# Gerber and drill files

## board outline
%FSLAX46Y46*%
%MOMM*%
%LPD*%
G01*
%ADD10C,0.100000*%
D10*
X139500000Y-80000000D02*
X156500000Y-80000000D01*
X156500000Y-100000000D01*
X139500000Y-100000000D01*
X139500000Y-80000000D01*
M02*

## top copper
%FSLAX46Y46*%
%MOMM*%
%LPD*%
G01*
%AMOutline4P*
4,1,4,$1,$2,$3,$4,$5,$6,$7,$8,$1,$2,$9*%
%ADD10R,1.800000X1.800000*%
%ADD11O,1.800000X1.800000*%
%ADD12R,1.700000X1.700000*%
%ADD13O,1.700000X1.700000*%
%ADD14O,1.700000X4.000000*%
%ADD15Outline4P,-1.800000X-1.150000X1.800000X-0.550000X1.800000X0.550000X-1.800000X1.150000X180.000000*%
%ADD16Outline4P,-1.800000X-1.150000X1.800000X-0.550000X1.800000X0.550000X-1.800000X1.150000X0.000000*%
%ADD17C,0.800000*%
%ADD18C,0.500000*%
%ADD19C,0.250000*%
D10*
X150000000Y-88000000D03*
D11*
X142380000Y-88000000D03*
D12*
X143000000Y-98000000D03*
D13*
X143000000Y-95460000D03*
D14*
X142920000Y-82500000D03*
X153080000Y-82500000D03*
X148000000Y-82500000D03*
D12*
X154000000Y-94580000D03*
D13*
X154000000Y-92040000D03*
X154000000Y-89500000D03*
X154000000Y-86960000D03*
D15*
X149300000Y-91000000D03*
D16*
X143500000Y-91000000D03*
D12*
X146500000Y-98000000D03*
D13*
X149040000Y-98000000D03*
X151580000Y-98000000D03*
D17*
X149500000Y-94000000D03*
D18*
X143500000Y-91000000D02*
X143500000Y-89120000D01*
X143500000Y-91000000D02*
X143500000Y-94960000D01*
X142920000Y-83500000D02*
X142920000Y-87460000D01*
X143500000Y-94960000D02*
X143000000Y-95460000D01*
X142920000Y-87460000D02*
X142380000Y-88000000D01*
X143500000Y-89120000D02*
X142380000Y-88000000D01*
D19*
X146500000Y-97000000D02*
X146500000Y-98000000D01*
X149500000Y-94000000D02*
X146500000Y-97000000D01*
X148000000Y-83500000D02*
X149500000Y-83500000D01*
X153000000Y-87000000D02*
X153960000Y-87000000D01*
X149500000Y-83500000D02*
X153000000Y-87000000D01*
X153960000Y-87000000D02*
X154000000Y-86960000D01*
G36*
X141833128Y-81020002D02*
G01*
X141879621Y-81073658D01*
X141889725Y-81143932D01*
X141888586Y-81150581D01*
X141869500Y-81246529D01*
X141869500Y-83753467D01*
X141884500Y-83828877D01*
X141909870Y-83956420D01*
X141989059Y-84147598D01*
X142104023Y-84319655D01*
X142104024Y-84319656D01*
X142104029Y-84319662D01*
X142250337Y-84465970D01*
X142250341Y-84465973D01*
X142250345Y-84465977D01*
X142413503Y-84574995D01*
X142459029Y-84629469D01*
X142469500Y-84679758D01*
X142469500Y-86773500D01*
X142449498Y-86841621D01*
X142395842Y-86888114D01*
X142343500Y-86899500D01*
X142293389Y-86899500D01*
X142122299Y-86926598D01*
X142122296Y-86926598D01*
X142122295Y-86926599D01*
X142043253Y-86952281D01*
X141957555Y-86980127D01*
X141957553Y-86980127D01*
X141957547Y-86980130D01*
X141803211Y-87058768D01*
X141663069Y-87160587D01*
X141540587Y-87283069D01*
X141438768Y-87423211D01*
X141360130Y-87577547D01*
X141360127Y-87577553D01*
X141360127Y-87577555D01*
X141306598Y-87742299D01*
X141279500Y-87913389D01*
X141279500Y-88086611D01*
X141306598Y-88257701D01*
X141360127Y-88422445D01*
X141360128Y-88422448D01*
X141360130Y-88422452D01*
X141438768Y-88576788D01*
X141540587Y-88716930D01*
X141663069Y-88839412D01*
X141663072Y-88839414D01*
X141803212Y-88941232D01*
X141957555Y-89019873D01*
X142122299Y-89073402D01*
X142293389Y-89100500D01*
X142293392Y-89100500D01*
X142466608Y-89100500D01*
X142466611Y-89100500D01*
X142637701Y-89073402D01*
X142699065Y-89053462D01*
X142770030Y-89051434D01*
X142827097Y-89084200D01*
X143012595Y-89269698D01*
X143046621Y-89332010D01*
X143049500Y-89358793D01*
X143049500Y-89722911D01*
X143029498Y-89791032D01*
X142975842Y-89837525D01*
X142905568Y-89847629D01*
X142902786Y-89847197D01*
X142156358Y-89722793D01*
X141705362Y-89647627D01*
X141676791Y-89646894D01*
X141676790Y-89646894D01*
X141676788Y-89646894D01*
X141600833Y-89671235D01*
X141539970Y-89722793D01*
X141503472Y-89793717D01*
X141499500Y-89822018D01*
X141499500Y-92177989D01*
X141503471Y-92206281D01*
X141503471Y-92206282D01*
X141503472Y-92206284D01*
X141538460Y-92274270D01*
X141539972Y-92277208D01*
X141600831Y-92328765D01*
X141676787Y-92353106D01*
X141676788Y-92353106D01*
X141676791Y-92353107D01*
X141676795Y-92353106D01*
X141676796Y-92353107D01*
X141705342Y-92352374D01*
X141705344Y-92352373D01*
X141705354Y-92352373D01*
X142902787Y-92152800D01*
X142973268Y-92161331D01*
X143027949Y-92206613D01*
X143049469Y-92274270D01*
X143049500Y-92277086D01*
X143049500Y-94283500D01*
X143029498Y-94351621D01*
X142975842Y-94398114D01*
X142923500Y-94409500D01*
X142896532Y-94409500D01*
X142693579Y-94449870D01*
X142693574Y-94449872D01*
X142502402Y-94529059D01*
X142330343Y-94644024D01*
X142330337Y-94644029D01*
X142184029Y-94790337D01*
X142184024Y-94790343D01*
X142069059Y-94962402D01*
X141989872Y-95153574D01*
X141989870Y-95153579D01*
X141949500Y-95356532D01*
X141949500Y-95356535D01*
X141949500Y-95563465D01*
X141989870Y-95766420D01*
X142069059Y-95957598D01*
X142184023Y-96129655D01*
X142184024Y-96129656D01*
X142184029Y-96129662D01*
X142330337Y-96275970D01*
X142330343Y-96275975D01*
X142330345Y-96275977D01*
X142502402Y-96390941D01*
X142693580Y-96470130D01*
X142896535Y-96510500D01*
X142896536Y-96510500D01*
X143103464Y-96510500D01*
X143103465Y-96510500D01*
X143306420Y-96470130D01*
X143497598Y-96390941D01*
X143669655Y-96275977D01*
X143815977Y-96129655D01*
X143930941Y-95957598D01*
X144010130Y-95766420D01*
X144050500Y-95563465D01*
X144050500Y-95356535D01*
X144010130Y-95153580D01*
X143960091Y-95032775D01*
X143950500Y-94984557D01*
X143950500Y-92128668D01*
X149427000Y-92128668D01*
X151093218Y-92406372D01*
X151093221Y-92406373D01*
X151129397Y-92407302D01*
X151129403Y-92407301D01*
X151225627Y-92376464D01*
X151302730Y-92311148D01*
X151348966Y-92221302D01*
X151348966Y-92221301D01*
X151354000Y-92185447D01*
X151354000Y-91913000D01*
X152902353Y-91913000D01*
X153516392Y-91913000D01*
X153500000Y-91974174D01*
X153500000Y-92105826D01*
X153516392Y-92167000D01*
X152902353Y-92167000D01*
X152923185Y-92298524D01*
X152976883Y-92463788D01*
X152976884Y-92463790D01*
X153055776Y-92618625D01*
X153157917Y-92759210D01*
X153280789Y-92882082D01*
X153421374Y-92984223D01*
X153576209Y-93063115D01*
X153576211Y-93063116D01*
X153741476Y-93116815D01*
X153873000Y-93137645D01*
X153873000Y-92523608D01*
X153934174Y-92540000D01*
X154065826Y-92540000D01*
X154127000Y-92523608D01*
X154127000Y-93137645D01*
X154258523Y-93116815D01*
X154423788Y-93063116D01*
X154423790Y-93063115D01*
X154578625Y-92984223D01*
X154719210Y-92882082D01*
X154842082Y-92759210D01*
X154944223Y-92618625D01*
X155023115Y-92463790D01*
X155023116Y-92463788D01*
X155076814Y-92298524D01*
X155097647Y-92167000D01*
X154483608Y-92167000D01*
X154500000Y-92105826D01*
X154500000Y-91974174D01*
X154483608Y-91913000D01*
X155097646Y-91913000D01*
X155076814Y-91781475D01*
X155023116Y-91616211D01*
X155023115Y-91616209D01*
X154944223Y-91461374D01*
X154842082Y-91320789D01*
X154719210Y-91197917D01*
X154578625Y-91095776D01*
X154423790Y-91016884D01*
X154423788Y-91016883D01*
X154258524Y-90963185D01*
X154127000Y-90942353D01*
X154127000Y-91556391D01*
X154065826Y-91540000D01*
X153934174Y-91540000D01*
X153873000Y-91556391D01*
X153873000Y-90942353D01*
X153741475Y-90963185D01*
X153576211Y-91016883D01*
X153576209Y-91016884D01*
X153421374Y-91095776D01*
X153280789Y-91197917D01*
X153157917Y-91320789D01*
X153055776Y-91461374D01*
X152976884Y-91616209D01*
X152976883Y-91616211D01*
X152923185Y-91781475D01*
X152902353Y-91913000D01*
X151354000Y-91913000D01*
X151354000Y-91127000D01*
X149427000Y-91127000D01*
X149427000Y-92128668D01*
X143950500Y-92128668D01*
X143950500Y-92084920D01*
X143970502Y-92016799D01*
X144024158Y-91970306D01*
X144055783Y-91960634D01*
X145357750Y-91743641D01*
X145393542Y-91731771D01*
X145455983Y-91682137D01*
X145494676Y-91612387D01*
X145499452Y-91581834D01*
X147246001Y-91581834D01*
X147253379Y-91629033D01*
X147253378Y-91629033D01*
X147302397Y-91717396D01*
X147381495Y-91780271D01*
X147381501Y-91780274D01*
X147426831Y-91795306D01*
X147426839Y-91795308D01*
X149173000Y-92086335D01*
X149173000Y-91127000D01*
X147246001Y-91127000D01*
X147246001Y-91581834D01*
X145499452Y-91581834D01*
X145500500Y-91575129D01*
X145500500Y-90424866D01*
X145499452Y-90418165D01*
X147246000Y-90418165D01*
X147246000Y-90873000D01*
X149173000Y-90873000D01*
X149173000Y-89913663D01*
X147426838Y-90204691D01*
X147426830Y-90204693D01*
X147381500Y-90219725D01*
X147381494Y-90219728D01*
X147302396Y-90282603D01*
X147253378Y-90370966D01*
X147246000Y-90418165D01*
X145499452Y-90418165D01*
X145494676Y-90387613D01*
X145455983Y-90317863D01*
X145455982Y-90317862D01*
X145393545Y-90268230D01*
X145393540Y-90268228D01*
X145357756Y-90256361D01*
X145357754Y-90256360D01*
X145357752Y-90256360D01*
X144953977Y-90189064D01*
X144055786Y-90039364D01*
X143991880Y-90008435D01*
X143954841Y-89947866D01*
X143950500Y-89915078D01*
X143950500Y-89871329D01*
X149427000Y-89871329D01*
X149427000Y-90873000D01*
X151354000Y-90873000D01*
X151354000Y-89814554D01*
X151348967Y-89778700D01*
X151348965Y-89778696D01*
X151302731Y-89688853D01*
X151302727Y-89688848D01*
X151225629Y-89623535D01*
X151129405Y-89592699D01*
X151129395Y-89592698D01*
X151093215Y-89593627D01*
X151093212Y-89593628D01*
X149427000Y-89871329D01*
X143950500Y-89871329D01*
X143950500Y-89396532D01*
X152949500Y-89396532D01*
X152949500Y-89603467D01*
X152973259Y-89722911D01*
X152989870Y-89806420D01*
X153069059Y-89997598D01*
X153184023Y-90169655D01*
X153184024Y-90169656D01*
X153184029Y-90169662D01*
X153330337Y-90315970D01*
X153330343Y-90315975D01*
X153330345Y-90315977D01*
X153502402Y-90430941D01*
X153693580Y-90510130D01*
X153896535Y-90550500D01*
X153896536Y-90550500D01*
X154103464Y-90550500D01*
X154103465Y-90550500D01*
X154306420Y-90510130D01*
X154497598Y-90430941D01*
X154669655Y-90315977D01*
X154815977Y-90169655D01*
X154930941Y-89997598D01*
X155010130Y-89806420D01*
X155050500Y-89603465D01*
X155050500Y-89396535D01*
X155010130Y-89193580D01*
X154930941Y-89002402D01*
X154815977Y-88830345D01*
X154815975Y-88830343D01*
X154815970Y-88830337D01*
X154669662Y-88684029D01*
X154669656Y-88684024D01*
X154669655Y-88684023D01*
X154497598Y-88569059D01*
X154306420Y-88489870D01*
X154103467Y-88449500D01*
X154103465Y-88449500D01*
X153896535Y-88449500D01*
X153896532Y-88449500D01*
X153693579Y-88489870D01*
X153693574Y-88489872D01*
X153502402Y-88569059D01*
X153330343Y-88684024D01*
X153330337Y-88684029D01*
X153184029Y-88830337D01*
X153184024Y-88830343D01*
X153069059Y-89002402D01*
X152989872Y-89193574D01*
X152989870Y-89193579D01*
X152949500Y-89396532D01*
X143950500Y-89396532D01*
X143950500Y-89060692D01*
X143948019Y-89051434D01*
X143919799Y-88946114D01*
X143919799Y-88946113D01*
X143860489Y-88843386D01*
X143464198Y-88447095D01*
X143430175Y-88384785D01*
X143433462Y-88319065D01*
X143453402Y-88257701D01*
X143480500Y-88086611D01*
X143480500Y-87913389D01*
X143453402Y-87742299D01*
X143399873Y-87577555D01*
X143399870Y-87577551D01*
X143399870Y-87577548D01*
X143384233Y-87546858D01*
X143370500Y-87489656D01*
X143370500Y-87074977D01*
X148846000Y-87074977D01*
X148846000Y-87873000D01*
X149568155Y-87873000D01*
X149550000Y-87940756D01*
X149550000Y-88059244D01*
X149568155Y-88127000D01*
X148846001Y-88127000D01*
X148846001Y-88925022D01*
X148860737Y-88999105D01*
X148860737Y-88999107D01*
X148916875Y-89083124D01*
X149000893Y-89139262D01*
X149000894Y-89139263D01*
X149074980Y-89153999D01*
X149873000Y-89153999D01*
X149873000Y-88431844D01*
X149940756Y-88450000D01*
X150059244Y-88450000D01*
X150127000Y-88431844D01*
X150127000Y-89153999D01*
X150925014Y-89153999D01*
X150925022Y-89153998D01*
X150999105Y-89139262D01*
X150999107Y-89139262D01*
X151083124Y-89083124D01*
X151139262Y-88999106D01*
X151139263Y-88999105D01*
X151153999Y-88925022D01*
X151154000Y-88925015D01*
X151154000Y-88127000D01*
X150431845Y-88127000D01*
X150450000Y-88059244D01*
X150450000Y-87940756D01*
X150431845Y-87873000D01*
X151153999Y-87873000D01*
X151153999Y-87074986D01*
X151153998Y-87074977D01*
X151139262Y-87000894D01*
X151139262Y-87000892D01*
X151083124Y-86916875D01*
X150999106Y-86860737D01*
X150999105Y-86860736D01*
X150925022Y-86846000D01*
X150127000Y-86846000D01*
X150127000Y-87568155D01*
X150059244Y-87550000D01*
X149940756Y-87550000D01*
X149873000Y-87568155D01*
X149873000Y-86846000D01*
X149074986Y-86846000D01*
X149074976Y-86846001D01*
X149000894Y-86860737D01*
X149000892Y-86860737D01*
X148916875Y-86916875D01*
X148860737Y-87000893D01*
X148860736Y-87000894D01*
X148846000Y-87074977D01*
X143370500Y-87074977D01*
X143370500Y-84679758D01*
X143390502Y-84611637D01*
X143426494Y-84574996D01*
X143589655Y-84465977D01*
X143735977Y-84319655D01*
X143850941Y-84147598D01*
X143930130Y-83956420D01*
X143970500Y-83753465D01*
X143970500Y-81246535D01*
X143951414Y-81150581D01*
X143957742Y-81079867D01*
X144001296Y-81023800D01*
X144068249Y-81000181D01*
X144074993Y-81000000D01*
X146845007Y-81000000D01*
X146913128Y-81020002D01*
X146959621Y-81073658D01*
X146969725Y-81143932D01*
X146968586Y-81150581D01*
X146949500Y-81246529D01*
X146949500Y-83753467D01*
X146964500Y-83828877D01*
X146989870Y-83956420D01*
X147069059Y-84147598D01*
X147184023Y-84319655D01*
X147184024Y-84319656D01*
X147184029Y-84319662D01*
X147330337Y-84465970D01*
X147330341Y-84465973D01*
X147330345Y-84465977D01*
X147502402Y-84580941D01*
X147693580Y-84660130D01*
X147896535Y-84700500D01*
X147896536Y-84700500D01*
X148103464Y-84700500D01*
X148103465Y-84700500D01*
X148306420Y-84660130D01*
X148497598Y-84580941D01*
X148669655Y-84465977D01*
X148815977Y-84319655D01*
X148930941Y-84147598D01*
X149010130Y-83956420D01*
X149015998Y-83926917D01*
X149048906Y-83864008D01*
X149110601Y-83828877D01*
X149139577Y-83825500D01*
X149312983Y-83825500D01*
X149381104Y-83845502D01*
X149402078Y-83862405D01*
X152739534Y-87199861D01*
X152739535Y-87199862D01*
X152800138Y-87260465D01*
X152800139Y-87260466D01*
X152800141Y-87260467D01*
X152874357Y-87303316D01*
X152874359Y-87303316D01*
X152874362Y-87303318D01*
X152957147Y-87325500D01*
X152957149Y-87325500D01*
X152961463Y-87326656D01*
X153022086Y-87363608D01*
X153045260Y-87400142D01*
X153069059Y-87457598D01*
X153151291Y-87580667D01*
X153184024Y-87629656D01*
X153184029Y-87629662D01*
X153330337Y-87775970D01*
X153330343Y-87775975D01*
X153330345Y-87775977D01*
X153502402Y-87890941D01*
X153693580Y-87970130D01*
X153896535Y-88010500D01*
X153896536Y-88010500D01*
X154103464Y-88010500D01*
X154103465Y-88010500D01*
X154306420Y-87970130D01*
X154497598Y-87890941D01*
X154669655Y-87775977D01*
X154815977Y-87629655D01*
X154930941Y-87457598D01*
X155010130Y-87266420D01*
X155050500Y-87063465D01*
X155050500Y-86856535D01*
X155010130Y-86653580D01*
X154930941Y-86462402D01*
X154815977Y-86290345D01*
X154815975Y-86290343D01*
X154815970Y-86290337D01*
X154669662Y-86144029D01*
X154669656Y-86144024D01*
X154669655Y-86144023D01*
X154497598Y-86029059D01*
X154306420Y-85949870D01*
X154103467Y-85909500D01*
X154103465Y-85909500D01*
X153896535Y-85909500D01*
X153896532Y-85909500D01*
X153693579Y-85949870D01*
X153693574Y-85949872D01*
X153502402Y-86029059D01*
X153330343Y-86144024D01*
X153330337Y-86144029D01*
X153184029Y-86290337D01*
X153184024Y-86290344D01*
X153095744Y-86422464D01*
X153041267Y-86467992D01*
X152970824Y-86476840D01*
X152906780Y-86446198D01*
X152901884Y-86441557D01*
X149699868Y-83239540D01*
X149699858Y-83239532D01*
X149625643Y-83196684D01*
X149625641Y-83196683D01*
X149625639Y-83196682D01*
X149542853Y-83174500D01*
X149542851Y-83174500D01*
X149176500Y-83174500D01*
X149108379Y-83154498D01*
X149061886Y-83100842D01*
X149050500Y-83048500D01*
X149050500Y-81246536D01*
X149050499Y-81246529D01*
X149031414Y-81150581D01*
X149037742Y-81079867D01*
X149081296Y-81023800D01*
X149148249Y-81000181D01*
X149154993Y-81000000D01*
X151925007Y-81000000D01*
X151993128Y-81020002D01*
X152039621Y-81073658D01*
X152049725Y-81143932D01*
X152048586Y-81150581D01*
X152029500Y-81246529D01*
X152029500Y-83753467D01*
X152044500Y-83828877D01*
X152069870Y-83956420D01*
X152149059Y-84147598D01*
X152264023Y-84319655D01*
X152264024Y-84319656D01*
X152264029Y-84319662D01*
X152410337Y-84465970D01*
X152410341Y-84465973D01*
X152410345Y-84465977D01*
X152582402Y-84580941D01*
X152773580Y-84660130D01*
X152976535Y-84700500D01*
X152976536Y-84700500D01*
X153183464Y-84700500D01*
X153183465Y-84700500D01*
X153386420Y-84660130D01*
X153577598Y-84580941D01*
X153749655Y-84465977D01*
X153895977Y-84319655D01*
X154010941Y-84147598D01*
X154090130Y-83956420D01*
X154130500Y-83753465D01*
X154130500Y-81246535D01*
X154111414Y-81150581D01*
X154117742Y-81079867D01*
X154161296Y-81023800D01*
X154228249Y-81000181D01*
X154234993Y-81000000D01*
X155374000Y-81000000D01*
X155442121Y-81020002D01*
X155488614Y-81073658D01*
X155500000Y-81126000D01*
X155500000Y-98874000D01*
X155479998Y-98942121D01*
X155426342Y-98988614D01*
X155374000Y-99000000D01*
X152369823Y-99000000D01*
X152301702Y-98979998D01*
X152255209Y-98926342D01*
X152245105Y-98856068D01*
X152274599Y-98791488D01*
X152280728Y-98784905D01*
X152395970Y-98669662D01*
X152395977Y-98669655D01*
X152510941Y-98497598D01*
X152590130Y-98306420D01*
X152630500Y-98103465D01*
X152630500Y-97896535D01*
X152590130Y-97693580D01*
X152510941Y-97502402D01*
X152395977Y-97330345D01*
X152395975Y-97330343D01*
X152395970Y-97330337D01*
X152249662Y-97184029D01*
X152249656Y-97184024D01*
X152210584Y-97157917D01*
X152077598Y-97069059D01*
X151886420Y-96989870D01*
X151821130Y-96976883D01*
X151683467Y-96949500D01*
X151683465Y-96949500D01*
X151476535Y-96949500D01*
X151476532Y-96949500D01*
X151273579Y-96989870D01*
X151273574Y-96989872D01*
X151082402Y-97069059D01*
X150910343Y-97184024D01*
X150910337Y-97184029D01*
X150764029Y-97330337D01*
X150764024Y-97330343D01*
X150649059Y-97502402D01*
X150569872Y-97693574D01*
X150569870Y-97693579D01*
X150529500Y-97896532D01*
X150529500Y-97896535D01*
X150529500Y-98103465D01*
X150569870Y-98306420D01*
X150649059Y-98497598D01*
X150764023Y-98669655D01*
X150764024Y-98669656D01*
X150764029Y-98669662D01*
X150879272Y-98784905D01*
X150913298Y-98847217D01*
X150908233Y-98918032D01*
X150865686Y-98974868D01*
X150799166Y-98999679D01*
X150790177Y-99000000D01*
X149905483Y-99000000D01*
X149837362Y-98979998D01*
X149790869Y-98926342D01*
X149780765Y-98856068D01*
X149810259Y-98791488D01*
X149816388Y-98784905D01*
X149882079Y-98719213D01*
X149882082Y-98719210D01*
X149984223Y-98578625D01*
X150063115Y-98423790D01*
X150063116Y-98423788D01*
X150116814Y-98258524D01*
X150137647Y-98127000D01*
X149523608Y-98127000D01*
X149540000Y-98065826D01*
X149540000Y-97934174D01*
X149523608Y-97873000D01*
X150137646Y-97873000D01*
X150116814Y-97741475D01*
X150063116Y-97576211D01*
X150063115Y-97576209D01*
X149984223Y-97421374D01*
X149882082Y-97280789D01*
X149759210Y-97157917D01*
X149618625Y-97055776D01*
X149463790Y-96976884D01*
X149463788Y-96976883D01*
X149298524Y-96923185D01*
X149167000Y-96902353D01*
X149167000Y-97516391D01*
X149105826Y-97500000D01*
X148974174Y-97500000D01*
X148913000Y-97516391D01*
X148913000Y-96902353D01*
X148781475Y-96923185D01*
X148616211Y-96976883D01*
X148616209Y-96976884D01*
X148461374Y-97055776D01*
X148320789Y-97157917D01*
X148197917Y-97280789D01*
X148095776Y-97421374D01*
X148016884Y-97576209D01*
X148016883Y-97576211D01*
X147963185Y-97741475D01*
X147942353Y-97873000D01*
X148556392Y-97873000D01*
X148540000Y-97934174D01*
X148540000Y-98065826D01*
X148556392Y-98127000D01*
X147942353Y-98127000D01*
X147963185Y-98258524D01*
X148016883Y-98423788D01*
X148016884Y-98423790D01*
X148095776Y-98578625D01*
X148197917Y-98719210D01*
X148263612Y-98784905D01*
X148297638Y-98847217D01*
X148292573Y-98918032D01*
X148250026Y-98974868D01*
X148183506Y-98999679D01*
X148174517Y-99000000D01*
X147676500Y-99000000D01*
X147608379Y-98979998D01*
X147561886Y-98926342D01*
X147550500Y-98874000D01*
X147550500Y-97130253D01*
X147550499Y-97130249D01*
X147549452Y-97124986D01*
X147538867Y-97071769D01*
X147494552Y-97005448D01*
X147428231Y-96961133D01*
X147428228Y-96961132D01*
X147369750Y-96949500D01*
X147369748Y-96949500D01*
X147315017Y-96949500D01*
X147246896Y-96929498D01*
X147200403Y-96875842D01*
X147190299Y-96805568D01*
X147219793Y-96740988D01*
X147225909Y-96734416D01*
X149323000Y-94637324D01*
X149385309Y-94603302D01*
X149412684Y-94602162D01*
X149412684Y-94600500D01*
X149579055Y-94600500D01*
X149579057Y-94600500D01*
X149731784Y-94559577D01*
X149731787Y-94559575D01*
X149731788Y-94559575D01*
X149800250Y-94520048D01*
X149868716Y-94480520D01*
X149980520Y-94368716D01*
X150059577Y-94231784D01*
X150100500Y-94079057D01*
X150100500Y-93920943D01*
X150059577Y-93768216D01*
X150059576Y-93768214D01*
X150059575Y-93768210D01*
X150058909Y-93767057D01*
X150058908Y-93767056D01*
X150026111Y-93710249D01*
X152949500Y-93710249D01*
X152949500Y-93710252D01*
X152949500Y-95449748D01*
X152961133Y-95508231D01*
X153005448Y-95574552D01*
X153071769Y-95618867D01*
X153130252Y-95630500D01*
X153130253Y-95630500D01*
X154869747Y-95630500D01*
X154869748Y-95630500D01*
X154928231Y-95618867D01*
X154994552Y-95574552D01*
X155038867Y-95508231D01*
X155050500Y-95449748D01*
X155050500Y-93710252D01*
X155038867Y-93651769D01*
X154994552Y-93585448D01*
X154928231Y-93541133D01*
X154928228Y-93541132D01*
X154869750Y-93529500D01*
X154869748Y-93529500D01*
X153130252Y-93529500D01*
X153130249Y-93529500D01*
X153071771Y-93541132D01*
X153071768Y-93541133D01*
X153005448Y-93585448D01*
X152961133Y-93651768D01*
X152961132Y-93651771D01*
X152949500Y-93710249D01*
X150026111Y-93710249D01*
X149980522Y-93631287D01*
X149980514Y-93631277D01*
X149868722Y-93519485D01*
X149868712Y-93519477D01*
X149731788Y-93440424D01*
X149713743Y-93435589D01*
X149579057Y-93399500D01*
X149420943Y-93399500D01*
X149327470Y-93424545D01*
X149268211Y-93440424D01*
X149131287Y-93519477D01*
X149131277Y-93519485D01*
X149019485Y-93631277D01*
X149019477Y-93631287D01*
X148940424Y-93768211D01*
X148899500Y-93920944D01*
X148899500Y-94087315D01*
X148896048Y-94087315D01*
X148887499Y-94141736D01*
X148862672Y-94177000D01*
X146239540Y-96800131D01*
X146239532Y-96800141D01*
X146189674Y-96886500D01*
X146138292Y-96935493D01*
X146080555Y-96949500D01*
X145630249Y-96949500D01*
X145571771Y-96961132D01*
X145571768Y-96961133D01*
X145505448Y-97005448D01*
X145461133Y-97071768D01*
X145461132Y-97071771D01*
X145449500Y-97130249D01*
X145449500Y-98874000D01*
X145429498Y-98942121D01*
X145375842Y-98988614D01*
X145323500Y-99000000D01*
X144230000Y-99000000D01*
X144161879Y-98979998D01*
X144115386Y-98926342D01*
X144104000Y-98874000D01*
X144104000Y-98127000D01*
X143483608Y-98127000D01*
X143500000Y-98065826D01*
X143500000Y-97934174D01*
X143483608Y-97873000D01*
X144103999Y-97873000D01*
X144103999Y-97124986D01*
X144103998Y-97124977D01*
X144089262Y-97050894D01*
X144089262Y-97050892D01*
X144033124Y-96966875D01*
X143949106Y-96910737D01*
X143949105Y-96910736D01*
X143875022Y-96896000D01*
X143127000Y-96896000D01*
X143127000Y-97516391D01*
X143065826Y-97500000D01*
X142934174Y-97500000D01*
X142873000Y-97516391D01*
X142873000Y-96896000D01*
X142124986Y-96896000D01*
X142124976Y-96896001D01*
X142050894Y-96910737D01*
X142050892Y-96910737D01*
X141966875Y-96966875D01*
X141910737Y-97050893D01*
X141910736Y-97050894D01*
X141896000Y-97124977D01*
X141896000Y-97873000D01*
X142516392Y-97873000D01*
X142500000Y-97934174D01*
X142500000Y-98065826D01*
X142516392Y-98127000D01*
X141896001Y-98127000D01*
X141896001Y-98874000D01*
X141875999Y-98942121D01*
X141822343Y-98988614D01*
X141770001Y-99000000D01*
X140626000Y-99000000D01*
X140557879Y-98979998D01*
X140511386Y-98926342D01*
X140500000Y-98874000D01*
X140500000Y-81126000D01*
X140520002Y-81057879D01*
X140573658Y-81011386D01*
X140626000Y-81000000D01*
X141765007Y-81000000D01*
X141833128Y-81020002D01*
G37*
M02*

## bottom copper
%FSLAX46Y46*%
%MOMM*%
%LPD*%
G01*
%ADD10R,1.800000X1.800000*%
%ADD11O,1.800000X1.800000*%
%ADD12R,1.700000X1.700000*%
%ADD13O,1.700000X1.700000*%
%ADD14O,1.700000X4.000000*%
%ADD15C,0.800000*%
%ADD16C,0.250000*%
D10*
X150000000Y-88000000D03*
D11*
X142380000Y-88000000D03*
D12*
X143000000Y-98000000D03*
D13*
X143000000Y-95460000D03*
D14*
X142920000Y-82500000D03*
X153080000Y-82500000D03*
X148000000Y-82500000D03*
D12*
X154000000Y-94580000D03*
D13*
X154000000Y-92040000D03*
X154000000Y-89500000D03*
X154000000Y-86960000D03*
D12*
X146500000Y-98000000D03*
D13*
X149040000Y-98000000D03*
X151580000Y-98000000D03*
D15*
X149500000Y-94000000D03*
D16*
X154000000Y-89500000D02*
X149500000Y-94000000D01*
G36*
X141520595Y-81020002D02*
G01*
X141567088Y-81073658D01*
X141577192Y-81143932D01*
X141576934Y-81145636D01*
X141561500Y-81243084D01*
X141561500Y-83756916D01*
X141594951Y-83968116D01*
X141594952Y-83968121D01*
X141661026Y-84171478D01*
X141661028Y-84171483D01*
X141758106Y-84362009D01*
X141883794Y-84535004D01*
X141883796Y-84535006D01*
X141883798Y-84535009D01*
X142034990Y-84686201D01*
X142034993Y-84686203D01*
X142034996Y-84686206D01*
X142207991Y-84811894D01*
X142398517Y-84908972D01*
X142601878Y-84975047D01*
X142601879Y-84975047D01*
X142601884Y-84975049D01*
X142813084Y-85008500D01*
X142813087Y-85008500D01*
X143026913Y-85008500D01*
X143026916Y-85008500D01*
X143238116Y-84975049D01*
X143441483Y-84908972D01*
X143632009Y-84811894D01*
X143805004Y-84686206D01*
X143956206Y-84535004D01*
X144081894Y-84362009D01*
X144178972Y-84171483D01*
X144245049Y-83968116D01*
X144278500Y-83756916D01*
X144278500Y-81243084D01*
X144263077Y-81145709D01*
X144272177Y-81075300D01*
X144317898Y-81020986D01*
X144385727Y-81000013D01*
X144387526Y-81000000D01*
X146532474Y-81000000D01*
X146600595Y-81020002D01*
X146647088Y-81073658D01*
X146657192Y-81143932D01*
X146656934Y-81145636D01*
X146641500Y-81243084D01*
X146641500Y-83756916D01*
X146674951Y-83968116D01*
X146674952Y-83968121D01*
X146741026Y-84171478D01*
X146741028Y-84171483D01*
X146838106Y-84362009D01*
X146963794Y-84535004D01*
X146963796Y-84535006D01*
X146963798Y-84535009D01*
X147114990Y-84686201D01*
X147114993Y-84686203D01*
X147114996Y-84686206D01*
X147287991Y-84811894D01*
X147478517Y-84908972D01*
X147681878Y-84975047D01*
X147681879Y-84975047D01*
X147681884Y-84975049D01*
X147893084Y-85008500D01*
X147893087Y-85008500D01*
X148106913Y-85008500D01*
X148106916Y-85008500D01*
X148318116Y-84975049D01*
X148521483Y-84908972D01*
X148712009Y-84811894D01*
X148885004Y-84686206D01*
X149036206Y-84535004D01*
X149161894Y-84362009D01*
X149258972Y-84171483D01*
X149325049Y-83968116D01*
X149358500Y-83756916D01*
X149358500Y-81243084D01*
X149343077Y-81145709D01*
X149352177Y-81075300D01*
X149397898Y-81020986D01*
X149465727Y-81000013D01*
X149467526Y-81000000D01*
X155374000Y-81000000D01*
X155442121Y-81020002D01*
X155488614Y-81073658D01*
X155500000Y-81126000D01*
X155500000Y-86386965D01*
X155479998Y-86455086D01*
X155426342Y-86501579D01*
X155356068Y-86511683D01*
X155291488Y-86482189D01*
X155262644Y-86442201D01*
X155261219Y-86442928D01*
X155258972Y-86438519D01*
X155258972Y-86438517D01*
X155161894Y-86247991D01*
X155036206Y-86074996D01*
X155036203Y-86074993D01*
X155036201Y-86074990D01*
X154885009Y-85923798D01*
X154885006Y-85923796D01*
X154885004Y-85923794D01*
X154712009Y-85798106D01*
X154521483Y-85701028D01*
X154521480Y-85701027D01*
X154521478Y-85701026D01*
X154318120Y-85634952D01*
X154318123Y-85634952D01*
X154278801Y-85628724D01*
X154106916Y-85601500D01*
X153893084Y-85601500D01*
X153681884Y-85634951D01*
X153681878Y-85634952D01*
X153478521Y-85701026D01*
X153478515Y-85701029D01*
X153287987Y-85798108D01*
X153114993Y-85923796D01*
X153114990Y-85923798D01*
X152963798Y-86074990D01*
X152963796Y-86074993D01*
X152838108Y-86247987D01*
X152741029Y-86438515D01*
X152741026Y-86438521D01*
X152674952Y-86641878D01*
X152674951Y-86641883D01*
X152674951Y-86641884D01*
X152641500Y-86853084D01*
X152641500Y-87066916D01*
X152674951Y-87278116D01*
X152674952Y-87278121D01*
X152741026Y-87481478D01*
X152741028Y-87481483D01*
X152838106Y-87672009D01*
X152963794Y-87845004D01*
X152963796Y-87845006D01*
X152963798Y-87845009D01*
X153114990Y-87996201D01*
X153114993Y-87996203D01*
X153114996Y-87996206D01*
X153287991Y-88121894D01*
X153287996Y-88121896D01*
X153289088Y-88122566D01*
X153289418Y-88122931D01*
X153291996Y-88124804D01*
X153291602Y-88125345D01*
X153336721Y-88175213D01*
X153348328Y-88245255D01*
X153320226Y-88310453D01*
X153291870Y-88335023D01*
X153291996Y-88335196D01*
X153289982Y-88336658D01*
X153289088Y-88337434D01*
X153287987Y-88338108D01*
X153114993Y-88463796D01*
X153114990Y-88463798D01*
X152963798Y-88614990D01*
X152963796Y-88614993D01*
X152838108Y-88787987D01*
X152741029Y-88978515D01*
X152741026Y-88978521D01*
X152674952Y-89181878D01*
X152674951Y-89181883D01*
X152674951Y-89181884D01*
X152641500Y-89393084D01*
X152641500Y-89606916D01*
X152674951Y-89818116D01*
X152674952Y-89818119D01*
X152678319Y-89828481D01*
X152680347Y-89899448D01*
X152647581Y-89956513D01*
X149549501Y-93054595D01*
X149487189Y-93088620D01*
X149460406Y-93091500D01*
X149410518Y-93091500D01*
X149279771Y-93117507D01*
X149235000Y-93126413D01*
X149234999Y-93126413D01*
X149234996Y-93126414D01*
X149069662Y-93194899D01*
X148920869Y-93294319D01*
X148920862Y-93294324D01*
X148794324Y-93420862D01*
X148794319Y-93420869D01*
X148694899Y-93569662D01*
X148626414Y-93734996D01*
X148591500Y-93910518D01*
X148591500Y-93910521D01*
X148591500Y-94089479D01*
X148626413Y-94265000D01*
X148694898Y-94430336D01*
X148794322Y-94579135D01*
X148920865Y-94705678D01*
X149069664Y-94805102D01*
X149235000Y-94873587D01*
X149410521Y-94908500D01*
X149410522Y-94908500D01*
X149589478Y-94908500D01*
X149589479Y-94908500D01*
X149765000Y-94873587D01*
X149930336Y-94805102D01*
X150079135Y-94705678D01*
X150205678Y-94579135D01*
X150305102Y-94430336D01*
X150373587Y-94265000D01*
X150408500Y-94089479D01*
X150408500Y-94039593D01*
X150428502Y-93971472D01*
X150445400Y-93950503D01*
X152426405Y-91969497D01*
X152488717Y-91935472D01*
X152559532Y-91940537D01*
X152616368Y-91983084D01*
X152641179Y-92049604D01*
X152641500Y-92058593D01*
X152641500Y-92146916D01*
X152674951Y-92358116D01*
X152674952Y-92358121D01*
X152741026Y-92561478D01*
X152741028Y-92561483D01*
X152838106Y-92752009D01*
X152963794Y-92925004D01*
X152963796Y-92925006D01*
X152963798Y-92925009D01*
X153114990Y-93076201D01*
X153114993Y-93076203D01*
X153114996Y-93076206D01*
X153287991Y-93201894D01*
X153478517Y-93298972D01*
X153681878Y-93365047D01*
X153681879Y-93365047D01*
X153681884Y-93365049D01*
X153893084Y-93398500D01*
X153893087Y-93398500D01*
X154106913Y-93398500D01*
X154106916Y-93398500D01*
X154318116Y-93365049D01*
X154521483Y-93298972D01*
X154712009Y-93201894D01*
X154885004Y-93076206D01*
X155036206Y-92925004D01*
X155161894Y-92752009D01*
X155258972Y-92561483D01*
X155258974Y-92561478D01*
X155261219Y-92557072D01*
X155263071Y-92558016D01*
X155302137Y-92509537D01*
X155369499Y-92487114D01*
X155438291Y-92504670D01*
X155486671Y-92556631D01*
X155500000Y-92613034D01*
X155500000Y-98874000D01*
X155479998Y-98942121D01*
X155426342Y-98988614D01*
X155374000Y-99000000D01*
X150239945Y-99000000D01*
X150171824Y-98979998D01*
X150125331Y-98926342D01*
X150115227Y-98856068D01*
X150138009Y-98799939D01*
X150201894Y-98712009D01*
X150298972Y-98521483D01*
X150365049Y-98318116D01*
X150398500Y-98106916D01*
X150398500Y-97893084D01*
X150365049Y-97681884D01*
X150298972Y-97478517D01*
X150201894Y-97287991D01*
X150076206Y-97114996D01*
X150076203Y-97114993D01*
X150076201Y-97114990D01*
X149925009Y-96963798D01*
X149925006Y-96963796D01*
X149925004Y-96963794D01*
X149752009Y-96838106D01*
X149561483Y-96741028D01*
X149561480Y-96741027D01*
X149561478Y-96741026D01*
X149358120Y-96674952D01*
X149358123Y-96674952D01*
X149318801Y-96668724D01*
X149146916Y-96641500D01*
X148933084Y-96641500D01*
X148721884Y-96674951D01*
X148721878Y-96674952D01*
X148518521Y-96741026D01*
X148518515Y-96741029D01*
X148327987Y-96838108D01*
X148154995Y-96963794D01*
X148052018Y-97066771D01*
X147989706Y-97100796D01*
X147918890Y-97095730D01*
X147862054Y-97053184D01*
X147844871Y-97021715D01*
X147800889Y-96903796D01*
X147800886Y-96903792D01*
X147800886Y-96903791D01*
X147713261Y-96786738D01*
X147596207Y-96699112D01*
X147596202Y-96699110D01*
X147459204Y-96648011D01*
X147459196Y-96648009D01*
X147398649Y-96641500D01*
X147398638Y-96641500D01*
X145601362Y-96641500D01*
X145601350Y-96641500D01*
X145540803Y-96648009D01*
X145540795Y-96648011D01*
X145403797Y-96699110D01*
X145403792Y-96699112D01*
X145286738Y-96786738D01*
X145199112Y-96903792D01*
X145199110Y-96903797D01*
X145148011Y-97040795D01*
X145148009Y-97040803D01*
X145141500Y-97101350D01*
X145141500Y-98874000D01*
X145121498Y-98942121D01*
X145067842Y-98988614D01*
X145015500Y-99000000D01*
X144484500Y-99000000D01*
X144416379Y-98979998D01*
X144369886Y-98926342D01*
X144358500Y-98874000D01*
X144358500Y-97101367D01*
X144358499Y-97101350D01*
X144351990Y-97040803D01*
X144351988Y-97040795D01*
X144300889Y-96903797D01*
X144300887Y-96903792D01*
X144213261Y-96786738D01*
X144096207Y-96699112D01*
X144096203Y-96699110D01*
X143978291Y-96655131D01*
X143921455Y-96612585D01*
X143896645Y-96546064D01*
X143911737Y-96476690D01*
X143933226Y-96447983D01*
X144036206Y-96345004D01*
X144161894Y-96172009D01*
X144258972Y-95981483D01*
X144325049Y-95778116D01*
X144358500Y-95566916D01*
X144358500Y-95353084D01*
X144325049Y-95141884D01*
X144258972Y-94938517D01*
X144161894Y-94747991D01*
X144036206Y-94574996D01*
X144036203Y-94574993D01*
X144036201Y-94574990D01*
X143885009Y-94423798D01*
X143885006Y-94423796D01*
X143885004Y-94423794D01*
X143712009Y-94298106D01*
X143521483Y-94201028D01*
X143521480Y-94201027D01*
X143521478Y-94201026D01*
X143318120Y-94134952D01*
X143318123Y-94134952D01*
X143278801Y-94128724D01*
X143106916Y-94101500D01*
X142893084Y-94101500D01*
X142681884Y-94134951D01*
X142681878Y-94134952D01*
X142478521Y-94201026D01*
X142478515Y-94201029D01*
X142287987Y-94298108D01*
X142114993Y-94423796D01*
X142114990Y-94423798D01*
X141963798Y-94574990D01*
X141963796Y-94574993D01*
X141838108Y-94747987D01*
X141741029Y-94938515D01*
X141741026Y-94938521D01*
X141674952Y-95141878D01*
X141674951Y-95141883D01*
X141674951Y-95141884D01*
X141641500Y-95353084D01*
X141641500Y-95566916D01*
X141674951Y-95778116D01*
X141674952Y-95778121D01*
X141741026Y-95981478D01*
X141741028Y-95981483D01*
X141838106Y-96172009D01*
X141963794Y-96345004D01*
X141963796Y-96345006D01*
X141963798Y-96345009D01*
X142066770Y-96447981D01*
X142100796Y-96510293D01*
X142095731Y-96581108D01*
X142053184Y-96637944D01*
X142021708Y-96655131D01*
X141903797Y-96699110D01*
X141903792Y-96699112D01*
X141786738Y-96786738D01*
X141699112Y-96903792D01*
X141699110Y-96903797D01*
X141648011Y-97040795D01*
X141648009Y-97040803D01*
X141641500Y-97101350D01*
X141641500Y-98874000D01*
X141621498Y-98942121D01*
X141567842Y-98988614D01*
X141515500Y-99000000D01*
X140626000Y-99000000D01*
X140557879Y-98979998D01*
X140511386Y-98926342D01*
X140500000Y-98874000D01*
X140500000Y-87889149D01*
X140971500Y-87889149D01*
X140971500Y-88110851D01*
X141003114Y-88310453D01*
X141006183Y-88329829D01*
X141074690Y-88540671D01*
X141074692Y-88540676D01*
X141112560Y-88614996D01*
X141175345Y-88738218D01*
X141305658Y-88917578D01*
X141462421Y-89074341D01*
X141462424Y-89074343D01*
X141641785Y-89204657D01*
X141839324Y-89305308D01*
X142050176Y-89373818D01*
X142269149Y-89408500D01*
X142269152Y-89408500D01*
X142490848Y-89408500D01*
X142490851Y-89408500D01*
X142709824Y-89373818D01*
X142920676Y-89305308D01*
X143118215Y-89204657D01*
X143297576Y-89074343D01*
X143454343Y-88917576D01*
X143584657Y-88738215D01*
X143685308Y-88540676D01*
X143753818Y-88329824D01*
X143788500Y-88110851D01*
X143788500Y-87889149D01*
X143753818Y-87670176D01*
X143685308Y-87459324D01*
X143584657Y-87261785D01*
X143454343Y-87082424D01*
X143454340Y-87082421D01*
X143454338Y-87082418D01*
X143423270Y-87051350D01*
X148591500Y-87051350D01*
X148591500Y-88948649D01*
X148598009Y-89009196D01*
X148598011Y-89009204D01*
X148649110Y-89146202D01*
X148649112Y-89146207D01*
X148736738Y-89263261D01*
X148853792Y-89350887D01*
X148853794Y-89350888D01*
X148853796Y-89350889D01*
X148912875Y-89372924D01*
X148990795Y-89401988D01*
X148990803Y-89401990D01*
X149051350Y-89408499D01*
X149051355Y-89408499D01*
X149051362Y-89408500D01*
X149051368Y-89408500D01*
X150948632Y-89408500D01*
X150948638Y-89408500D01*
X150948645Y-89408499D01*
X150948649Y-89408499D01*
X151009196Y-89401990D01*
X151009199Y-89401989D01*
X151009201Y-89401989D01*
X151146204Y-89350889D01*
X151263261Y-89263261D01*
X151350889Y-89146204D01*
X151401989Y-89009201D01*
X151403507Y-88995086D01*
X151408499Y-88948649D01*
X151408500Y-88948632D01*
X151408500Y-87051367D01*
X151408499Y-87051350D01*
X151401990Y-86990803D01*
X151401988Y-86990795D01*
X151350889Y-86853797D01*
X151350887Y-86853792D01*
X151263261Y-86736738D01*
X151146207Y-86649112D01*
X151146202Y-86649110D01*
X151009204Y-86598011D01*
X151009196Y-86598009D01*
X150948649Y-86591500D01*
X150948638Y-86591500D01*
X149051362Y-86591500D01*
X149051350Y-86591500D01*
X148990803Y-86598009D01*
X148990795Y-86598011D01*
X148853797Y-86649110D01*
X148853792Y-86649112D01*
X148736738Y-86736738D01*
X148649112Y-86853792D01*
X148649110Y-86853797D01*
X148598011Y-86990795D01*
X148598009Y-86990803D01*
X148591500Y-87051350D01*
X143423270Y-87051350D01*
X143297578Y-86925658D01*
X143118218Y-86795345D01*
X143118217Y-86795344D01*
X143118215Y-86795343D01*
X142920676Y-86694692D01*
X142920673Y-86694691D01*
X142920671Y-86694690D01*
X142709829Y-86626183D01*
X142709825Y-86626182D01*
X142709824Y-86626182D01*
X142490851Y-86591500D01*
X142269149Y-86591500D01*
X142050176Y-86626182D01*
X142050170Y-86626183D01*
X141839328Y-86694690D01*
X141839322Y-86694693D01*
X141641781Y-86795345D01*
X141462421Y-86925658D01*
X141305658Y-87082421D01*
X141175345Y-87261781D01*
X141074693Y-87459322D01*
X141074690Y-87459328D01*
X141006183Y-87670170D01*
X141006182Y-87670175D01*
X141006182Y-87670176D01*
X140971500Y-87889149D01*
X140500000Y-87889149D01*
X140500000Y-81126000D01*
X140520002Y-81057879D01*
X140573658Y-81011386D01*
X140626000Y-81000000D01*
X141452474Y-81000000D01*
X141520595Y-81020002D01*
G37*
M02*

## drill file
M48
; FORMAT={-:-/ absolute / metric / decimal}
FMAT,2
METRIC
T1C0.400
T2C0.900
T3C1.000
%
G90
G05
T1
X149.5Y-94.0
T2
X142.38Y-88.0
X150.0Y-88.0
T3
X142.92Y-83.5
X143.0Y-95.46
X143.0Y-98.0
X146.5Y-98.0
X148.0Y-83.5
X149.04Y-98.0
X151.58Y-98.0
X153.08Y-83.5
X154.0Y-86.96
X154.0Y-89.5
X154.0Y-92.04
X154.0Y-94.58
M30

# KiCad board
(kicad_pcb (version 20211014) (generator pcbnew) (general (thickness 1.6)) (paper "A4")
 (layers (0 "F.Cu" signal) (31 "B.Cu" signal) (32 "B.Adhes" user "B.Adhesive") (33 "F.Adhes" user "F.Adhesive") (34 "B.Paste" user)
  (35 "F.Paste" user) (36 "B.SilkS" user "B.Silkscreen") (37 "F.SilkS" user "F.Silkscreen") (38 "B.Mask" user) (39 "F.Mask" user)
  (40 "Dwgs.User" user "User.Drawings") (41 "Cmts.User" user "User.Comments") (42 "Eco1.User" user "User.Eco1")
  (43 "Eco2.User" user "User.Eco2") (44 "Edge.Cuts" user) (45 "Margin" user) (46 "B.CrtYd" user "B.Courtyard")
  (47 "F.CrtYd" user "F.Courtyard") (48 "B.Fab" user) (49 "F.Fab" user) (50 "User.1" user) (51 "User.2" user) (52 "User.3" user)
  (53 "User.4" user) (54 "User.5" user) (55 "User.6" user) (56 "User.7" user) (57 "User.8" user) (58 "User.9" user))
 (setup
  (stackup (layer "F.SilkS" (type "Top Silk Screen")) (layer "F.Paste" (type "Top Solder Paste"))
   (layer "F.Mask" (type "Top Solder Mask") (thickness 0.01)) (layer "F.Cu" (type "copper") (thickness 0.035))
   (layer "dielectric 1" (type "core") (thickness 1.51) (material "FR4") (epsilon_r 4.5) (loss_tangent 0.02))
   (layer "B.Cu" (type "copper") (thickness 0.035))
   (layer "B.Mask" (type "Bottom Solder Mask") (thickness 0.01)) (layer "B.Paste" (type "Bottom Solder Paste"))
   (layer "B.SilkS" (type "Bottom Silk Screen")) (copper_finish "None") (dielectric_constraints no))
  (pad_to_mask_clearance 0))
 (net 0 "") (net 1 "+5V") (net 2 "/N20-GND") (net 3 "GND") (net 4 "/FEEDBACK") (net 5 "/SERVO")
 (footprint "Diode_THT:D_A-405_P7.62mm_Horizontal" (layer "F.Cu") (at 150 88 180)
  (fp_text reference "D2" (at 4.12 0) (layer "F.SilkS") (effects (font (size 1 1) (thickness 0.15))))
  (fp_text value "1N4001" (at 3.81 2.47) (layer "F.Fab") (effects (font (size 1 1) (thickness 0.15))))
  (pad "1" thru_hole rect (at 0 0 180) (size 1.8 1.8) (drill 0.9) (layers *.Cu *.Mask) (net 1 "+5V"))
  (pad "2" thru_hole oval (at 7.62 0 180) (size 1.8 1.8) (drill 0.9) (layers *.Cu *.Mask) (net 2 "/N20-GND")))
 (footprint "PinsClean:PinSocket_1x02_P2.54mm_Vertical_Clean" (layer "F.Cu") (at 143 98 180)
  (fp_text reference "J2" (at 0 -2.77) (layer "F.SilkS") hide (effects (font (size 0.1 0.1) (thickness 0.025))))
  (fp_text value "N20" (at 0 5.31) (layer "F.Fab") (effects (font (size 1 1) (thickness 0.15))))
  (pad "1" thru_hole rect (at 0 0 180) (size 1.7 1.7) (drill 1) (layers *.Cu *.Mask) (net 1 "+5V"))
  (pad "2" thru_hole oval (at 0 2.54 180) (size 1.7 1.7) (drill 1) (layers *.Cu *.Mask) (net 2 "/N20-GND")))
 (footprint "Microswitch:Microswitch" (layer "F.Cu") (at 153.08 83.5 -90)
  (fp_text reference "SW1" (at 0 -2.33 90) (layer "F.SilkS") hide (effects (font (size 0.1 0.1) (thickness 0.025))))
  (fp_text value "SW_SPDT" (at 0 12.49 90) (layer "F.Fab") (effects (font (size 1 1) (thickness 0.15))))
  (pad "1" thru_hole oval (at 0 10.16 270) (size 4 1.7) (drill 1 (offset -1 0)) (layers *.Cu *.Mask) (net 2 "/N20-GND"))
  (pad "2" thru_hole oval (at 0 0 270) (size 4 1.7) (drill 1 (offset -1 0)) (layers *.Cu *.Mask) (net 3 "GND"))
  (pad "3" thru_hole oval (at 0 5.08 270) (size 4 1.7) (drill 1 (offset -1 0)) (layers *.Cu *.Mask) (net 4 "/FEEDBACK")))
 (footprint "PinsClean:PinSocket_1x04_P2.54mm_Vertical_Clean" (layer "F.Cu") (at 154 94.58 180)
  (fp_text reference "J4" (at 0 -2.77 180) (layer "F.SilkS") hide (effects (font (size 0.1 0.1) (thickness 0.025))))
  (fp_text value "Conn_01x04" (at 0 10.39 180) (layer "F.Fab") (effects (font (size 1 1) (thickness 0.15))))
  (pad "1" thru_hole rect (at 0 0 180) (size 1.7 1.7) (drill 1) (layers *.Cu *.Mask) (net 3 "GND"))
  (pad "2" thru_hole oval (at 0 2.54 180) (size 1.7 1.7) (drill 1) (layers *.Cu *.Mask) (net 1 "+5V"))
  (pad "3" thru_hole oval (at 0 5.08 180) (size 1.7 1.7) (drill 1) (layers *.Cu *.Mask) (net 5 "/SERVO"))
  (pad "4" thru_hole oval (at 0 7.62 180) (size 1.7 1.7) (drill 1) (layers *.Cu *.Mask) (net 4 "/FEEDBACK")))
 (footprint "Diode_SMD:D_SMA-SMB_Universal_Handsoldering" (layer "F.Cu") (at 146.4 91 180)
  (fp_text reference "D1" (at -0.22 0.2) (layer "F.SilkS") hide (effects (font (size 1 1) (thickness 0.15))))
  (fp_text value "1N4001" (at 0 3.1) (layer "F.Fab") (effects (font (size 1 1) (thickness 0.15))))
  (pad "1" smd trapezoid (at -2.9 0 180) (size 3.6 1.7) (rect_delta 0.6 0) (layers "F.Cu" "F.Paste" "F.Mask") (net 1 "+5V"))
  (pad "2" smd trapezoid (at 2.9 0) (size 3.6 1.7) (rect_delta 0.6 0) (layers "F.Cu" "F.Paste" "F.Mask") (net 2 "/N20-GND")))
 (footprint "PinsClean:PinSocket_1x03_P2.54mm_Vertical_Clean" (layer "F.Cu") (at 146.5 98 90)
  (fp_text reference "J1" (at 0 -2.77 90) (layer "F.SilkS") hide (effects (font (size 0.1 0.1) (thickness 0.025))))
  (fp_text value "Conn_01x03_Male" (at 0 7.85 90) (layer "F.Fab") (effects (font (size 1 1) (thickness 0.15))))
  (pad "1" thru_hole rect (at 0 0 90) (size 1.7 1.7) (drill 1) (layers *.Cu *.Mask) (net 5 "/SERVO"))
  (pad "2" thru_hole oval (at 0 2.54 90) (size 1.7 1.7) (drill 1) (layers *.Cu *.Mask) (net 1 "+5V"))
  (pad "3" thru_hole oval (at 0 5.08 90) (size 1.7 1.7) (drill 1) (layers *.Cu *.Mask) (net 3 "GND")))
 (gr_rect (start 139.5 80) (end 156.5 100) (layer "Edge.Cuts") (width 0.1) (fill none))
 (segment (start 143.5 91) (end 143.5 89.12) (width 0.5) (layer "F.Cu") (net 2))
 (segment (start 143.5 91) (end 143.5 94.96) (width 0.5) (layer "F.Cu") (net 2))
 (segment (start 142.92 83.5) (end 142.92 87.46) (width 0.5) (layer "F.Cu") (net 2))
 (segment (start 143.5 94.96) (end 143 95.46) (width 0.5) (layer "F.Cu") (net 2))
 (segment (start 142.92 87.46) (end 142.38 88) (width 0.5) (layer "F.Cu") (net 2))
 (segment (start 143.5 89.12) (end 142.38 88) (width 0.5) (layer "F.Cu") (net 2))
 (segment (start 146.5 97) (end 146.5 98) (width 0.25) (layer "F.Cu") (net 5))
 (segment (start 149.5 94) (end 146.5 97) (width 0.25) (layer "F.Cu") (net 5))
 (via (at 149.5 94) (size 0.8) (drill 0.4) (layers "F.Cu" "B.Cu") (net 5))
 (segment (start 154 89.5) (end 149.5 94) (width 0.25) (layer "B.Cu") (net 5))
 (segment (start 148 83.5) (end 149.5 83.5) (width 0.25) (layer "F.Cu") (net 4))
 (segment (start 153 87) (end 153.96 87) (width 0.25) (layer "F.Cu") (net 4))
 (segment (start 149.5 83.5) (end 153 87) (width 0.25) (layer "F.Cu") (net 4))
 (segment (start 153.96 87) (end 154 86.96) (width 0.25) (layer "F.Cu") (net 4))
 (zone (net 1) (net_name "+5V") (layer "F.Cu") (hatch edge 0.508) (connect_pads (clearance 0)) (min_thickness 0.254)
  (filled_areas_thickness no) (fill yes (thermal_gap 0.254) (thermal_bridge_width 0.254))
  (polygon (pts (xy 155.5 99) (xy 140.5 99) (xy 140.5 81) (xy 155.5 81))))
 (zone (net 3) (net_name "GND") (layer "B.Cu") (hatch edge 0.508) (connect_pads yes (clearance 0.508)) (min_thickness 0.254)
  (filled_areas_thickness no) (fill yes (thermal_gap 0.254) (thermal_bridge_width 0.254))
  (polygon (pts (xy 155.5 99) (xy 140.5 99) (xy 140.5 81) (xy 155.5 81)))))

